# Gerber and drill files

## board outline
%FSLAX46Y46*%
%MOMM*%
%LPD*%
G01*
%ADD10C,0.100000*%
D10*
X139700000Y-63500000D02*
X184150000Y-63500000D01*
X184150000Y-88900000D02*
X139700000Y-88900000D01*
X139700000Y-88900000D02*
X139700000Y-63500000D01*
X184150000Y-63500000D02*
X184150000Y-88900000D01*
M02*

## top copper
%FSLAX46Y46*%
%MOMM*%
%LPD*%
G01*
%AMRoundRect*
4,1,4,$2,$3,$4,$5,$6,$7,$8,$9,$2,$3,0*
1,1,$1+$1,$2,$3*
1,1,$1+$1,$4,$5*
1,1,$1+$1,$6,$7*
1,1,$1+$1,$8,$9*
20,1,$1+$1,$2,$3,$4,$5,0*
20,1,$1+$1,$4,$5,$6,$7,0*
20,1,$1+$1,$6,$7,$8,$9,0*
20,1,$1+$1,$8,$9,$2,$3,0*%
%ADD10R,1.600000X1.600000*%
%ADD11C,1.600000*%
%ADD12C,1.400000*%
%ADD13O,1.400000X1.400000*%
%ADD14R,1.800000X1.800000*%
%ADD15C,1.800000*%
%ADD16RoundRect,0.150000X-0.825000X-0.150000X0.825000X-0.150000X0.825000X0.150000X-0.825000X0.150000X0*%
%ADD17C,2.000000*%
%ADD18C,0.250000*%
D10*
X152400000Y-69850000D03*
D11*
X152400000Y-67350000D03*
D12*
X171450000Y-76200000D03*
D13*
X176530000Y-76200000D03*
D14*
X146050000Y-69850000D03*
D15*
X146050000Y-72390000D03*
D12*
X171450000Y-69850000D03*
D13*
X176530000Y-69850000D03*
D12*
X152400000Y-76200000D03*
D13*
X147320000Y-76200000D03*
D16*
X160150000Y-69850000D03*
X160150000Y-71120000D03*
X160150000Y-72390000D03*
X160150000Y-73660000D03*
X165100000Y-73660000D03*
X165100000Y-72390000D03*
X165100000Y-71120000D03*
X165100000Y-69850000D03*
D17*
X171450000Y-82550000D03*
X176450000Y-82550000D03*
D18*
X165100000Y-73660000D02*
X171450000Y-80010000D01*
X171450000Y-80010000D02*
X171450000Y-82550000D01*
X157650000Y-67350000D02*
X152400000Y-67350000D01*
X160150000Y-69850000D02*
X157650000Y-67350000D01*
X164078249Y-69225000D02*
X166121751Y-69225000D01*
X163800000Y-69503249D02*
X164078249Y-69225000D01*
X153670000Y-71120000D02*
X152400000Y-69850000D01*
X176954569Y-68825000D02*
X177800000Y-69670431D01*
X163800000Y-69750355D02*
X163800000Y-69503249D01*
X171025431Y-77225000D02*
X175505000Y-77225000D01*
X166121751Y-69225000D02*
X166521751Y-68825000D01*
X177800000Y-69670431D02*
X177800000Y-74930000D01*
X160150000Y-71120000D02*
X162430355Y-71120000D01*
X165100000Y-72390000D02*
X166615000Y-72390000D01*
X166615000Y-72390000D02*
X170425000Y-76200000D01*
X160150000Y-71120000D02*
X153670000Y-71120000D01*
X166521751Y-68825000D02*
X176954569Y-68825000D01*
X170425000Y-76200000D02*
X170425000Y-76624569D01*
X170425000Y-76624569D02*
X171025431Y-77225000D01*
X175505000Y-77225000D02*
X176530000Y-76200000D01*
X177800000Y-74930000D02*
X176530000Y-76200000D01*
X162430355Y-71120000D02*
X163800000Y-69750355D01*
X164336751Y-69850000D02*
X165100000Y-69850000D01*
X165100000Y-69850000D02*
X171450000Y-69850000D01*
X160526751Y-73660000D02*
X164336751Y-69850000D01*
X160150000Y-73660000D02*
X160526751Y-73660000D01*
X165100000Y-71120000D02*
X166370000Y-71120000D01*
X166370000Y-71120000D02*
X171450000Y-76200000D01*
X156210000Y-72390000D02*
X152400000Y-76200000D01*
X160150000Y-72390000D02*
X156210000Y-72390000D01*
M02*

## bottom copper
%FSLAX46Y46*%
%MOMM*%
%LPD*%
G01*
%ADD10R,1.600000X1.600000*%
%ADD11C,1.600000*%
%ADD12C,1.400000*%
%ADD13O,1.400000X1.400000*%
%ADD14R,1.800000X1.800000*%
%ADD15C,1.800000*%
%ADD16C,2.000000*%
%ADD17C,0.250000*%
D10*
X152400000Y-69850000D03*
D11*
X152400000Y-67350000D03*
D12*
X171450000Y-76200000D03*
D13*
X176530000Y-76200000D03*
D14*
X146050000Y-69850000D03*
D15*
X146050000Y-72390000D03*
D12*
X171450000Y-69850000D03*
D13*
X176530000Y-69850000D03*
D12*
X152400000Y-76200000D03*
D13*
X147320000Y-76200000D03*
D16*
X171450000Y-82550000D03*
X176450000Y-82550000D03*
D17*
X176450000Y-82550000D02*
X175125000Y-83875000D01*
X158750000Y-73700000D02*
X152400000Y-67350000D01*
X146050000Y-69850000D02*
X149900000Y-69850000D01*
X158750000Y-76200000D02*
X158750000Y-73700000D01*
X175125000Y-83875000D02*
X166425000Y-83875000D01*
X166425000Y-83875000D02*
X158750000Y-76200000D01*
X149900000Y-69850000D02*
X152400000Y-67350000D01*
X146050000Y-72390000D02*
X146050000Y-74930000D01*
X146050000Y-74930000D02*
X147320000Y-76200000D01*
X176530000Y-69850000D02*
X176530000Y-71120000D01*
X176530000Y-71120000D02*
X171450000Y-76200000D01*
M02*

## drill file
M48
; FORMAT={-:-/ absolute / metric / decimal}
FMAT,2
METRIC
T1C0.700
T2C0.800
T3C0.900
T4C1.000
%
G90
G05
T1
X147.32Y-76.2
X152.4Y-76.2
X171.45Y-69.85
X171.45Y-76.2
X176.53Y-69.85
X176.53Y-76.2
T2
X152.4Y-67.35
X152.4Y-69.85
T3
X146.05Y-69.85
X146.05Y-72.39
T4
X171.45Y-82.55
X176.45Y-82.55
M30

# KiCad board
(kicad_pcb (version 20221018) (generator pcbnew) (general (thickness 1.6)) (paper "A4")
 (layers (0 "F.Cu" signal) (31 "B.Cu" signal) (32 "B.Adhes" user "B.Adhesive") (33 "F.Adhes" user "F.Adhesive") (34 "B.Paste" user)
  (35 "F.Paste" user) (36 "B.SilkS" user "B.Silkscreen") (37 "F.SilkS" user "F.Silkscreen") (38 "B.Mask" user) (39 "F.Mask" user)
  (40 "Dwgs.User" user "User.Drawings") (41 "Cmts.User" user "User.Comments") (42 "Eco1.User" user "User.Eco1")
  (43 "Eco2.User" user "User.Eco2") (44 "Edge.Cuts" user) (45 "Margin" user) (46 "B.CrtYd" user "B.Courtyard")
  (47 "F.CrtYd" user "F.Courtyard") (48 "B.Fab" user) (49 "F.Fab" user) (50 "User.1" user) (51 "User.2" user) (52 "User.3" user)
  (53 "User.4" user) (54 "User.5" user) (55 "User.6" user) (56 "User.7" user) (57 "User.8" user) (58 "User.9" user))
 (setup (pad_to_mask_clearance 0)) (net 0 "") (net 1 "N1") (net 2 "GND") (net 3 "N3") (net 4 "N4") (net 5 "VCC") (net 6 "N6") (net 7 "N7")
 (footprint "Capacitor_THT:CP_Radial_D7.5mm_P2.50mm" (layer "F.Cu") (at 152.4 69.85 90)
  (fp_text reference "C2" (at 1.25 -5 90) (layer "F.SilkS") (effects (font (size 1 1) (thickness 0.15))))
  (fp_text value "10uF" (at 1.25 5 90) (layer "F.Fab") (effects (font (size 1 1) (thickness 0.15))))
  (pad "1" thru_hole rect (at 0 0 90) (size 1.6 1.6) (drill 0.8) (layers "*.Cu" "*.Mask") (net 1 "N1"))
  (pad "2" thru_hole circle (at 2.5 0 90) (size 1.6 1.6) (drill 0.8) (layers "*.Cu" "*.Mask") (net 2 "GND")))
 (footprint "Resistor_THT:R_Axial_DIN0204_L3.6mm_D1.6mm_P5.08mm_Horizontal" (layer "F.Cu") (at 171.45 76.2)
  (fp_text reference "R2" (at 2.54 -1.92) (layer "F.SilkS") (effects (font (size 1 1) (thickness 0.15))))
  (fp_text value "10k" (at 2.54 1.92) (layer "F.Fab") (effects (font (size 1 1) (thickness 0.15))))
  (pad "1" thru_hole circle (at 0 0) (size 1.4 1.4) (drill 0.7) (layers "*.Cu" "*.Mask") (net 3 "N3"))
  (pad "2" thru_hole oval (at 5.08 0) (size 1.4 1.4) (drill 0.7) (layers "*.Cu" "*.Mask") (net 1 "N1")))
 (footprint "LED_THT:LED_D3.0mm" (layer "F.Cu") (at 146.05 69.85 -90)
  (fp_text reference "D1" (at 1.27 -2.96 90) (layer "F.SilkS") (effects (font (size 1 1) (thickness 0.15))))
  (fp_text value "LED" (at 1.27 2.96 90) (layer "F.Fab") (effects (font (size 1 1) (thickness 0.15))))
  (pad "1" thru_hole rect (at 0 0 270) (size 1.8 1.8) (drill 0.9) (layers "*.Cu" "*.Mask") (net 2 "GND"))
  (pad "2" thru_hole circle (at 2.54 0 270) (size 1.8 1.8) (drill 0.9) (layers "*.Cu" "*.Mask") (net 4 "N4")))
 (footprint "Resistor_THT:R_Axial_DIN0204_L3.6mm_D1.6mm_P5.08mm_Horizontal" (layer "F.Cu") (at 171.45 69.85)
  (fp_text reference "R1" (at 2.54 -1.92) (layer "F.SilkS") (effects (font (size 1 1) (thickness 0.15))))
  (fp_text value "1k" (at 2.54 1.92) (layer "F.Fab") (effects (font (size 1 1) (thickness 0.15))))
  (pad "1" thru_hole circle (at 0 0) (size 1.4 1.4) (drill 0.7) (layers "*.Cu" "*.Mask") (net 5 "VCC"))
  (pad "2" thru_hole oval (at 5.08 0) (size 1.4 1.4) (drill 0.7) (layers "*.Cu" "*.Mask") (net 3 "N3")))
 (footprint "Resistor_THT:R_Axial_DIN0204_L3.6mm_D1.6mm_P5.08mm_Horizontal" (layer "F.Cu") (at 152.4 76.2 180)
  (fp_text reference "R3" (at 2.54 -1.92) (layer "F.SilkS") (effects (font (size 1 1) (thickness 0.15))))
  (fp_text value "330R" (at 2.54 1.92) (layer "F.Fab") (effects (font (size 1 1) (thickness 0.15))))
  (pad "1" thru_hole circle (at 0 0 180) (size 1.4 1.4) (drill 0.7) (layers "*.Cu" "*.Mask") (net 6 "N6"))
  (pad "2" thru_hole oval (at 5.08 0 180) (size 1.4 1.4) (drill 0.7) (layers "*.Cu" "*.Mask") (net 4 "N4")))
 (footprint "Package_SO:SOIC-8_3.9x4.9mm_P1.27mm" (layer "F.Cu") (at 162.625 71.755)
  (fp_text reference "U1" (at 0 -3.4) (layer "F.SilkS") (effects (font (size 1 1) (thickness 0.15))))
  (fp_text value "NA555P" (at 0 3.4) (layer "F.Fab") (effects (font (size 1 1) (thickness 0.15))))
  (pad "1" smd roundrect (at -2.475 -1.905) (size 1.95 0.6) (layers "F.Cu" "F.Paste" "F.Mask") (roundrect_rratio 0.25) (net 2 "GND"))
  (pad "2" smd roundrect (at -2.475 -0.635) (size 1.95 0.6) (layers "F.Cu" "F.Paste" "F.Mask") (roundrect_rratio 0.25) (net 1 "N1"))
  (pad "3" smd roundrect (at -2.475 0.635) (size 1.95 0.6) (layers "F.Cu" "F.Paste" "F.Mask") (roundrect_rratio 0.25) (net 6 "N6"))
  (pad "4" smd roundrect (at -2.475 1.905) (size 1.95 0.6) (layers "F.Cu" "F.Paste" "F.Mask") (roundrect_rratio 0.25) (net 5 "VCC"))
  (pad "5" smd roundrect (at 2.475 1.905) (size 1.95 0.6) (layers "F.Cu" "F.Paste" "F.Mask") (roundrect_rratio 0.25) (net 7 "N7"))
  (pad "6" smd roundrect (at 2.475 0.635) (size 1.95 0.6) (layers "F.Cu" "F.Paste" "F.Mask") (roundrect_rratio 0.25) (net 1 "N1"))
  (pad "7" smd roundrect (at 2.475 -0.635) (size 1.95 0.6) (layers "F.Cu" "F.Paste" "F.Mask") (roundrect_rratio 0.25) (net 3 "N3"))
  (pad "8" smd roundrect (at 2.475 -1.905) (size 1.95 0.6) (layers "F.Cu" "F.Paste" "F.Mask") (roundrect_rratio 0.25) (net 5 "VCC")))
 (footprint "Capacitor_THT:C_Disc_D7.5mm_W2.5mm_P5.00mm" (layer "F.Cu") (at 171.45 82.55)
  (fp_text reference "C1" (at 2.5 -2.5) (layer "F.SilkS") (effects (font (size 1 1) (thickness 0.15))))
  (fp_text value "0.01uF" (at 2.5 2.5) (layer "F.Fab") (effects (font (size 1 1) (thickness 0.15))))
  (pad "1" thru_hole circle (at 0 0) (size 2 2) (drill 1) (layers "*.Cu" "*.Mask") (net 7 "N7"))
  (pad "2" thru_hole circle (at 5 0) (size 2 2) (drill 1) (layers "*.Cu" "*.Mask") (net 2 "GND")))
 (gr_line (start 139.7 63.5) (end 184.15 63.5) (stroke (width 0.1) (type default)) (layer "Edge.Cuts"))
 (gr_line (start 184.15 88.9) (end 139.7 88.9) (stroke (width 0.1) (type default)) (layer "Edge.Cuts"))
 (gr_line (start 139.7 88.9) (end 139.7 63.5) (stroke (width 0.1) (type default)) (layer "Edge.Cuts"))
 (gr_line (start 184.15 63.5) (end 184.15 88.9) (stroke (width 0.1) (type default)) (layer "Edge.Cuts"))
 (segment (start 165.1 73.66) (end 171.45 80.01) (width 0.25) (layer "F.Cu") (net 7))
 (segment (start 171.45 80.01) (end 171.45 82.55) (width 0.25) (layer "F.Cu") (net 7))
 (segment (start 157.65 67.35) (end 152.4 67.35) (width 0.25) (layer "F.Cu") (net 2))
 (segment (start 160.15 69.85) (end 157.65 67.35) (width 0.25) (layer "F.Cu") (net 2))
 (segment (start 176.45 82.55) (end 175.125 83.875) (width 0.25) (layer "B.Cu") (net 2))
 (segment (start 158.75 73.7) (end 152.4 67.35) (width 0.25) (layer "B.Cu") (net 2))
 (segment (start 146.05 69.85) (end 149.9 69.85) (width 0.25) (layer "B.Cu") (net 2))
 (segment (start 158.75 76.2) (end 158.75 73.7) (width 0.25) (layer "B.Cu") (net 2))
 (segment (start 175.125 83.875) (end 166.425 83.875) (width 0.25) (layer "B.Cu") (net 2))
 (segment (start 166.425 83.875) (end 158.75 76.2) (width 0.25) (layer "B.Cu") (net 2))
 (segment (start 149.9 69.85) (end 152.4 67.35) (width 0.25) (layer "B.Cu") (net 2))
 (segment (start 164.078249 69.225) (end 166.121751 69.225) (width 0.25) (layer "F.Cu") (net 1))
 (segment (start 163.8 69.503249) (end 164.078249 69.225) (width 0.25) (layer "F.Cu") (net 1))
 (segment (start 153.67 71.12) (end 152.4 69.85) (width 0.25) (layer "F.Cu") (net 1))
 (segment (start 176.954569 68.825) (end 177.8 69.670431) (width 0.25) (layer "F.Cu") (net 1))
 (segment (start 163.8 69.750355) (end 163.8 69.503249) (width 0.25) (layer "F.Cu") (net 1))
 (segment (start 171.025431 77.225) (end 175.505 77.225) (width 0.25) (layer "F.Cu") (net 1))
 (segment (start 166.121751 69.225) (end 166.521751 68.825) (width 0.25) (layer "F.Cu") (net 1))
 (segment (start 177.8 69.670431) (end 177.8 74.93) (width 0.25) (layer "F.Cu") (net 1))
 (segment (start 160.15 71.12) (end 162.430355 71.12) (width 0.25) (layer "F.Cu") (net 1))
 (segment (start 165.1 72.39) (end 166.615 72.39) (width 0.25) (layer "F.Cu") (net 1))
 (segment (start 166.615 72.39) (end 170.425 76.2) (width 0.25) (layer "F.Cu") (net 1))
 (segment (start 160.15 71.12) (end 153.67 71.12) (width 0.25) (layer "F.Cu") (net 1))
 (segment (start 166.521751 68.825) (end 176.954569 68.825) (width 0.25) (layer "F.Cu") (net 1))
 (segment (start 170.425 76.2) (end 170.425 76.624569) (width 0.25) (layer "F.Cu") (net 1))
 (segment (start 170.425 76.624569) (end 171.025431 77.225) (width 0.25) (layer "F.Cu") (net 1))
 (segment (start 175.505 77.225) (end 176.53 76.2) (width 0.25) (layer "F.Cu") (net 1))
 (segment (start 177.8 74.93) (end 176.53 76.2) (width 0.25) (layer "F.Cu") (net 1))
 (segment (start 162.430355 71.12) (end 163.8 69.750355) (width 0.25) (layer "F.Cu") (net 1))
 (segment (start 146.05 72.39) (end 146.05 74.93) (width 0.25) (layer "B.Cu") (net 4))
 (segment (start 146.05 74.93) (end 147.32 76.2) (width 0.25) (layer "B.Cu") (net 4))
 (segment (start 164.336751 69.85) (end 165.1 69.85) (width 0.25) (layer "F.Cu") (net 5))
 (segment (start 165.1 69.85) (end 171.45 69.85) (width 0.25) (layer "F.Cu") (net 5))
 (segment (start 160.526751 73.66) (end 164.336751 69.85) (width 0.25) (layer "F.Cu") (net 5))
 (segment (start 160.15 73.66) (end 160.526751 73.66) (width 0.25) (layer "F.Cu") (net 5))
 (segment (start 165.1 71.12) (end 166.37 71.12) (width 0.25) (layer "F.Cu") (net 3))
 (segment (start 166.37 71.12) (end 171.45 76.2) (width 0.25) (layer "F.Cu") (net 3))
 (segment (start 176.53 69.85) (end 176.53 71.12) (width 0.25) (layer "B.Cu") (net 3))
 (segment (start 176.53 71.12) (end 171.45 76.2) (width 0.25) (layer "B.Cu") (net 3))
 (segment (start 156.21 72.39) (end 152.4 76.2) (width 0.25) (layer "F.Cu") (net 6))
 (segment (start 160.15 72.39) (end 156.21 72.39) (width 0.25) (layer "F.Cu") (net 6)))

